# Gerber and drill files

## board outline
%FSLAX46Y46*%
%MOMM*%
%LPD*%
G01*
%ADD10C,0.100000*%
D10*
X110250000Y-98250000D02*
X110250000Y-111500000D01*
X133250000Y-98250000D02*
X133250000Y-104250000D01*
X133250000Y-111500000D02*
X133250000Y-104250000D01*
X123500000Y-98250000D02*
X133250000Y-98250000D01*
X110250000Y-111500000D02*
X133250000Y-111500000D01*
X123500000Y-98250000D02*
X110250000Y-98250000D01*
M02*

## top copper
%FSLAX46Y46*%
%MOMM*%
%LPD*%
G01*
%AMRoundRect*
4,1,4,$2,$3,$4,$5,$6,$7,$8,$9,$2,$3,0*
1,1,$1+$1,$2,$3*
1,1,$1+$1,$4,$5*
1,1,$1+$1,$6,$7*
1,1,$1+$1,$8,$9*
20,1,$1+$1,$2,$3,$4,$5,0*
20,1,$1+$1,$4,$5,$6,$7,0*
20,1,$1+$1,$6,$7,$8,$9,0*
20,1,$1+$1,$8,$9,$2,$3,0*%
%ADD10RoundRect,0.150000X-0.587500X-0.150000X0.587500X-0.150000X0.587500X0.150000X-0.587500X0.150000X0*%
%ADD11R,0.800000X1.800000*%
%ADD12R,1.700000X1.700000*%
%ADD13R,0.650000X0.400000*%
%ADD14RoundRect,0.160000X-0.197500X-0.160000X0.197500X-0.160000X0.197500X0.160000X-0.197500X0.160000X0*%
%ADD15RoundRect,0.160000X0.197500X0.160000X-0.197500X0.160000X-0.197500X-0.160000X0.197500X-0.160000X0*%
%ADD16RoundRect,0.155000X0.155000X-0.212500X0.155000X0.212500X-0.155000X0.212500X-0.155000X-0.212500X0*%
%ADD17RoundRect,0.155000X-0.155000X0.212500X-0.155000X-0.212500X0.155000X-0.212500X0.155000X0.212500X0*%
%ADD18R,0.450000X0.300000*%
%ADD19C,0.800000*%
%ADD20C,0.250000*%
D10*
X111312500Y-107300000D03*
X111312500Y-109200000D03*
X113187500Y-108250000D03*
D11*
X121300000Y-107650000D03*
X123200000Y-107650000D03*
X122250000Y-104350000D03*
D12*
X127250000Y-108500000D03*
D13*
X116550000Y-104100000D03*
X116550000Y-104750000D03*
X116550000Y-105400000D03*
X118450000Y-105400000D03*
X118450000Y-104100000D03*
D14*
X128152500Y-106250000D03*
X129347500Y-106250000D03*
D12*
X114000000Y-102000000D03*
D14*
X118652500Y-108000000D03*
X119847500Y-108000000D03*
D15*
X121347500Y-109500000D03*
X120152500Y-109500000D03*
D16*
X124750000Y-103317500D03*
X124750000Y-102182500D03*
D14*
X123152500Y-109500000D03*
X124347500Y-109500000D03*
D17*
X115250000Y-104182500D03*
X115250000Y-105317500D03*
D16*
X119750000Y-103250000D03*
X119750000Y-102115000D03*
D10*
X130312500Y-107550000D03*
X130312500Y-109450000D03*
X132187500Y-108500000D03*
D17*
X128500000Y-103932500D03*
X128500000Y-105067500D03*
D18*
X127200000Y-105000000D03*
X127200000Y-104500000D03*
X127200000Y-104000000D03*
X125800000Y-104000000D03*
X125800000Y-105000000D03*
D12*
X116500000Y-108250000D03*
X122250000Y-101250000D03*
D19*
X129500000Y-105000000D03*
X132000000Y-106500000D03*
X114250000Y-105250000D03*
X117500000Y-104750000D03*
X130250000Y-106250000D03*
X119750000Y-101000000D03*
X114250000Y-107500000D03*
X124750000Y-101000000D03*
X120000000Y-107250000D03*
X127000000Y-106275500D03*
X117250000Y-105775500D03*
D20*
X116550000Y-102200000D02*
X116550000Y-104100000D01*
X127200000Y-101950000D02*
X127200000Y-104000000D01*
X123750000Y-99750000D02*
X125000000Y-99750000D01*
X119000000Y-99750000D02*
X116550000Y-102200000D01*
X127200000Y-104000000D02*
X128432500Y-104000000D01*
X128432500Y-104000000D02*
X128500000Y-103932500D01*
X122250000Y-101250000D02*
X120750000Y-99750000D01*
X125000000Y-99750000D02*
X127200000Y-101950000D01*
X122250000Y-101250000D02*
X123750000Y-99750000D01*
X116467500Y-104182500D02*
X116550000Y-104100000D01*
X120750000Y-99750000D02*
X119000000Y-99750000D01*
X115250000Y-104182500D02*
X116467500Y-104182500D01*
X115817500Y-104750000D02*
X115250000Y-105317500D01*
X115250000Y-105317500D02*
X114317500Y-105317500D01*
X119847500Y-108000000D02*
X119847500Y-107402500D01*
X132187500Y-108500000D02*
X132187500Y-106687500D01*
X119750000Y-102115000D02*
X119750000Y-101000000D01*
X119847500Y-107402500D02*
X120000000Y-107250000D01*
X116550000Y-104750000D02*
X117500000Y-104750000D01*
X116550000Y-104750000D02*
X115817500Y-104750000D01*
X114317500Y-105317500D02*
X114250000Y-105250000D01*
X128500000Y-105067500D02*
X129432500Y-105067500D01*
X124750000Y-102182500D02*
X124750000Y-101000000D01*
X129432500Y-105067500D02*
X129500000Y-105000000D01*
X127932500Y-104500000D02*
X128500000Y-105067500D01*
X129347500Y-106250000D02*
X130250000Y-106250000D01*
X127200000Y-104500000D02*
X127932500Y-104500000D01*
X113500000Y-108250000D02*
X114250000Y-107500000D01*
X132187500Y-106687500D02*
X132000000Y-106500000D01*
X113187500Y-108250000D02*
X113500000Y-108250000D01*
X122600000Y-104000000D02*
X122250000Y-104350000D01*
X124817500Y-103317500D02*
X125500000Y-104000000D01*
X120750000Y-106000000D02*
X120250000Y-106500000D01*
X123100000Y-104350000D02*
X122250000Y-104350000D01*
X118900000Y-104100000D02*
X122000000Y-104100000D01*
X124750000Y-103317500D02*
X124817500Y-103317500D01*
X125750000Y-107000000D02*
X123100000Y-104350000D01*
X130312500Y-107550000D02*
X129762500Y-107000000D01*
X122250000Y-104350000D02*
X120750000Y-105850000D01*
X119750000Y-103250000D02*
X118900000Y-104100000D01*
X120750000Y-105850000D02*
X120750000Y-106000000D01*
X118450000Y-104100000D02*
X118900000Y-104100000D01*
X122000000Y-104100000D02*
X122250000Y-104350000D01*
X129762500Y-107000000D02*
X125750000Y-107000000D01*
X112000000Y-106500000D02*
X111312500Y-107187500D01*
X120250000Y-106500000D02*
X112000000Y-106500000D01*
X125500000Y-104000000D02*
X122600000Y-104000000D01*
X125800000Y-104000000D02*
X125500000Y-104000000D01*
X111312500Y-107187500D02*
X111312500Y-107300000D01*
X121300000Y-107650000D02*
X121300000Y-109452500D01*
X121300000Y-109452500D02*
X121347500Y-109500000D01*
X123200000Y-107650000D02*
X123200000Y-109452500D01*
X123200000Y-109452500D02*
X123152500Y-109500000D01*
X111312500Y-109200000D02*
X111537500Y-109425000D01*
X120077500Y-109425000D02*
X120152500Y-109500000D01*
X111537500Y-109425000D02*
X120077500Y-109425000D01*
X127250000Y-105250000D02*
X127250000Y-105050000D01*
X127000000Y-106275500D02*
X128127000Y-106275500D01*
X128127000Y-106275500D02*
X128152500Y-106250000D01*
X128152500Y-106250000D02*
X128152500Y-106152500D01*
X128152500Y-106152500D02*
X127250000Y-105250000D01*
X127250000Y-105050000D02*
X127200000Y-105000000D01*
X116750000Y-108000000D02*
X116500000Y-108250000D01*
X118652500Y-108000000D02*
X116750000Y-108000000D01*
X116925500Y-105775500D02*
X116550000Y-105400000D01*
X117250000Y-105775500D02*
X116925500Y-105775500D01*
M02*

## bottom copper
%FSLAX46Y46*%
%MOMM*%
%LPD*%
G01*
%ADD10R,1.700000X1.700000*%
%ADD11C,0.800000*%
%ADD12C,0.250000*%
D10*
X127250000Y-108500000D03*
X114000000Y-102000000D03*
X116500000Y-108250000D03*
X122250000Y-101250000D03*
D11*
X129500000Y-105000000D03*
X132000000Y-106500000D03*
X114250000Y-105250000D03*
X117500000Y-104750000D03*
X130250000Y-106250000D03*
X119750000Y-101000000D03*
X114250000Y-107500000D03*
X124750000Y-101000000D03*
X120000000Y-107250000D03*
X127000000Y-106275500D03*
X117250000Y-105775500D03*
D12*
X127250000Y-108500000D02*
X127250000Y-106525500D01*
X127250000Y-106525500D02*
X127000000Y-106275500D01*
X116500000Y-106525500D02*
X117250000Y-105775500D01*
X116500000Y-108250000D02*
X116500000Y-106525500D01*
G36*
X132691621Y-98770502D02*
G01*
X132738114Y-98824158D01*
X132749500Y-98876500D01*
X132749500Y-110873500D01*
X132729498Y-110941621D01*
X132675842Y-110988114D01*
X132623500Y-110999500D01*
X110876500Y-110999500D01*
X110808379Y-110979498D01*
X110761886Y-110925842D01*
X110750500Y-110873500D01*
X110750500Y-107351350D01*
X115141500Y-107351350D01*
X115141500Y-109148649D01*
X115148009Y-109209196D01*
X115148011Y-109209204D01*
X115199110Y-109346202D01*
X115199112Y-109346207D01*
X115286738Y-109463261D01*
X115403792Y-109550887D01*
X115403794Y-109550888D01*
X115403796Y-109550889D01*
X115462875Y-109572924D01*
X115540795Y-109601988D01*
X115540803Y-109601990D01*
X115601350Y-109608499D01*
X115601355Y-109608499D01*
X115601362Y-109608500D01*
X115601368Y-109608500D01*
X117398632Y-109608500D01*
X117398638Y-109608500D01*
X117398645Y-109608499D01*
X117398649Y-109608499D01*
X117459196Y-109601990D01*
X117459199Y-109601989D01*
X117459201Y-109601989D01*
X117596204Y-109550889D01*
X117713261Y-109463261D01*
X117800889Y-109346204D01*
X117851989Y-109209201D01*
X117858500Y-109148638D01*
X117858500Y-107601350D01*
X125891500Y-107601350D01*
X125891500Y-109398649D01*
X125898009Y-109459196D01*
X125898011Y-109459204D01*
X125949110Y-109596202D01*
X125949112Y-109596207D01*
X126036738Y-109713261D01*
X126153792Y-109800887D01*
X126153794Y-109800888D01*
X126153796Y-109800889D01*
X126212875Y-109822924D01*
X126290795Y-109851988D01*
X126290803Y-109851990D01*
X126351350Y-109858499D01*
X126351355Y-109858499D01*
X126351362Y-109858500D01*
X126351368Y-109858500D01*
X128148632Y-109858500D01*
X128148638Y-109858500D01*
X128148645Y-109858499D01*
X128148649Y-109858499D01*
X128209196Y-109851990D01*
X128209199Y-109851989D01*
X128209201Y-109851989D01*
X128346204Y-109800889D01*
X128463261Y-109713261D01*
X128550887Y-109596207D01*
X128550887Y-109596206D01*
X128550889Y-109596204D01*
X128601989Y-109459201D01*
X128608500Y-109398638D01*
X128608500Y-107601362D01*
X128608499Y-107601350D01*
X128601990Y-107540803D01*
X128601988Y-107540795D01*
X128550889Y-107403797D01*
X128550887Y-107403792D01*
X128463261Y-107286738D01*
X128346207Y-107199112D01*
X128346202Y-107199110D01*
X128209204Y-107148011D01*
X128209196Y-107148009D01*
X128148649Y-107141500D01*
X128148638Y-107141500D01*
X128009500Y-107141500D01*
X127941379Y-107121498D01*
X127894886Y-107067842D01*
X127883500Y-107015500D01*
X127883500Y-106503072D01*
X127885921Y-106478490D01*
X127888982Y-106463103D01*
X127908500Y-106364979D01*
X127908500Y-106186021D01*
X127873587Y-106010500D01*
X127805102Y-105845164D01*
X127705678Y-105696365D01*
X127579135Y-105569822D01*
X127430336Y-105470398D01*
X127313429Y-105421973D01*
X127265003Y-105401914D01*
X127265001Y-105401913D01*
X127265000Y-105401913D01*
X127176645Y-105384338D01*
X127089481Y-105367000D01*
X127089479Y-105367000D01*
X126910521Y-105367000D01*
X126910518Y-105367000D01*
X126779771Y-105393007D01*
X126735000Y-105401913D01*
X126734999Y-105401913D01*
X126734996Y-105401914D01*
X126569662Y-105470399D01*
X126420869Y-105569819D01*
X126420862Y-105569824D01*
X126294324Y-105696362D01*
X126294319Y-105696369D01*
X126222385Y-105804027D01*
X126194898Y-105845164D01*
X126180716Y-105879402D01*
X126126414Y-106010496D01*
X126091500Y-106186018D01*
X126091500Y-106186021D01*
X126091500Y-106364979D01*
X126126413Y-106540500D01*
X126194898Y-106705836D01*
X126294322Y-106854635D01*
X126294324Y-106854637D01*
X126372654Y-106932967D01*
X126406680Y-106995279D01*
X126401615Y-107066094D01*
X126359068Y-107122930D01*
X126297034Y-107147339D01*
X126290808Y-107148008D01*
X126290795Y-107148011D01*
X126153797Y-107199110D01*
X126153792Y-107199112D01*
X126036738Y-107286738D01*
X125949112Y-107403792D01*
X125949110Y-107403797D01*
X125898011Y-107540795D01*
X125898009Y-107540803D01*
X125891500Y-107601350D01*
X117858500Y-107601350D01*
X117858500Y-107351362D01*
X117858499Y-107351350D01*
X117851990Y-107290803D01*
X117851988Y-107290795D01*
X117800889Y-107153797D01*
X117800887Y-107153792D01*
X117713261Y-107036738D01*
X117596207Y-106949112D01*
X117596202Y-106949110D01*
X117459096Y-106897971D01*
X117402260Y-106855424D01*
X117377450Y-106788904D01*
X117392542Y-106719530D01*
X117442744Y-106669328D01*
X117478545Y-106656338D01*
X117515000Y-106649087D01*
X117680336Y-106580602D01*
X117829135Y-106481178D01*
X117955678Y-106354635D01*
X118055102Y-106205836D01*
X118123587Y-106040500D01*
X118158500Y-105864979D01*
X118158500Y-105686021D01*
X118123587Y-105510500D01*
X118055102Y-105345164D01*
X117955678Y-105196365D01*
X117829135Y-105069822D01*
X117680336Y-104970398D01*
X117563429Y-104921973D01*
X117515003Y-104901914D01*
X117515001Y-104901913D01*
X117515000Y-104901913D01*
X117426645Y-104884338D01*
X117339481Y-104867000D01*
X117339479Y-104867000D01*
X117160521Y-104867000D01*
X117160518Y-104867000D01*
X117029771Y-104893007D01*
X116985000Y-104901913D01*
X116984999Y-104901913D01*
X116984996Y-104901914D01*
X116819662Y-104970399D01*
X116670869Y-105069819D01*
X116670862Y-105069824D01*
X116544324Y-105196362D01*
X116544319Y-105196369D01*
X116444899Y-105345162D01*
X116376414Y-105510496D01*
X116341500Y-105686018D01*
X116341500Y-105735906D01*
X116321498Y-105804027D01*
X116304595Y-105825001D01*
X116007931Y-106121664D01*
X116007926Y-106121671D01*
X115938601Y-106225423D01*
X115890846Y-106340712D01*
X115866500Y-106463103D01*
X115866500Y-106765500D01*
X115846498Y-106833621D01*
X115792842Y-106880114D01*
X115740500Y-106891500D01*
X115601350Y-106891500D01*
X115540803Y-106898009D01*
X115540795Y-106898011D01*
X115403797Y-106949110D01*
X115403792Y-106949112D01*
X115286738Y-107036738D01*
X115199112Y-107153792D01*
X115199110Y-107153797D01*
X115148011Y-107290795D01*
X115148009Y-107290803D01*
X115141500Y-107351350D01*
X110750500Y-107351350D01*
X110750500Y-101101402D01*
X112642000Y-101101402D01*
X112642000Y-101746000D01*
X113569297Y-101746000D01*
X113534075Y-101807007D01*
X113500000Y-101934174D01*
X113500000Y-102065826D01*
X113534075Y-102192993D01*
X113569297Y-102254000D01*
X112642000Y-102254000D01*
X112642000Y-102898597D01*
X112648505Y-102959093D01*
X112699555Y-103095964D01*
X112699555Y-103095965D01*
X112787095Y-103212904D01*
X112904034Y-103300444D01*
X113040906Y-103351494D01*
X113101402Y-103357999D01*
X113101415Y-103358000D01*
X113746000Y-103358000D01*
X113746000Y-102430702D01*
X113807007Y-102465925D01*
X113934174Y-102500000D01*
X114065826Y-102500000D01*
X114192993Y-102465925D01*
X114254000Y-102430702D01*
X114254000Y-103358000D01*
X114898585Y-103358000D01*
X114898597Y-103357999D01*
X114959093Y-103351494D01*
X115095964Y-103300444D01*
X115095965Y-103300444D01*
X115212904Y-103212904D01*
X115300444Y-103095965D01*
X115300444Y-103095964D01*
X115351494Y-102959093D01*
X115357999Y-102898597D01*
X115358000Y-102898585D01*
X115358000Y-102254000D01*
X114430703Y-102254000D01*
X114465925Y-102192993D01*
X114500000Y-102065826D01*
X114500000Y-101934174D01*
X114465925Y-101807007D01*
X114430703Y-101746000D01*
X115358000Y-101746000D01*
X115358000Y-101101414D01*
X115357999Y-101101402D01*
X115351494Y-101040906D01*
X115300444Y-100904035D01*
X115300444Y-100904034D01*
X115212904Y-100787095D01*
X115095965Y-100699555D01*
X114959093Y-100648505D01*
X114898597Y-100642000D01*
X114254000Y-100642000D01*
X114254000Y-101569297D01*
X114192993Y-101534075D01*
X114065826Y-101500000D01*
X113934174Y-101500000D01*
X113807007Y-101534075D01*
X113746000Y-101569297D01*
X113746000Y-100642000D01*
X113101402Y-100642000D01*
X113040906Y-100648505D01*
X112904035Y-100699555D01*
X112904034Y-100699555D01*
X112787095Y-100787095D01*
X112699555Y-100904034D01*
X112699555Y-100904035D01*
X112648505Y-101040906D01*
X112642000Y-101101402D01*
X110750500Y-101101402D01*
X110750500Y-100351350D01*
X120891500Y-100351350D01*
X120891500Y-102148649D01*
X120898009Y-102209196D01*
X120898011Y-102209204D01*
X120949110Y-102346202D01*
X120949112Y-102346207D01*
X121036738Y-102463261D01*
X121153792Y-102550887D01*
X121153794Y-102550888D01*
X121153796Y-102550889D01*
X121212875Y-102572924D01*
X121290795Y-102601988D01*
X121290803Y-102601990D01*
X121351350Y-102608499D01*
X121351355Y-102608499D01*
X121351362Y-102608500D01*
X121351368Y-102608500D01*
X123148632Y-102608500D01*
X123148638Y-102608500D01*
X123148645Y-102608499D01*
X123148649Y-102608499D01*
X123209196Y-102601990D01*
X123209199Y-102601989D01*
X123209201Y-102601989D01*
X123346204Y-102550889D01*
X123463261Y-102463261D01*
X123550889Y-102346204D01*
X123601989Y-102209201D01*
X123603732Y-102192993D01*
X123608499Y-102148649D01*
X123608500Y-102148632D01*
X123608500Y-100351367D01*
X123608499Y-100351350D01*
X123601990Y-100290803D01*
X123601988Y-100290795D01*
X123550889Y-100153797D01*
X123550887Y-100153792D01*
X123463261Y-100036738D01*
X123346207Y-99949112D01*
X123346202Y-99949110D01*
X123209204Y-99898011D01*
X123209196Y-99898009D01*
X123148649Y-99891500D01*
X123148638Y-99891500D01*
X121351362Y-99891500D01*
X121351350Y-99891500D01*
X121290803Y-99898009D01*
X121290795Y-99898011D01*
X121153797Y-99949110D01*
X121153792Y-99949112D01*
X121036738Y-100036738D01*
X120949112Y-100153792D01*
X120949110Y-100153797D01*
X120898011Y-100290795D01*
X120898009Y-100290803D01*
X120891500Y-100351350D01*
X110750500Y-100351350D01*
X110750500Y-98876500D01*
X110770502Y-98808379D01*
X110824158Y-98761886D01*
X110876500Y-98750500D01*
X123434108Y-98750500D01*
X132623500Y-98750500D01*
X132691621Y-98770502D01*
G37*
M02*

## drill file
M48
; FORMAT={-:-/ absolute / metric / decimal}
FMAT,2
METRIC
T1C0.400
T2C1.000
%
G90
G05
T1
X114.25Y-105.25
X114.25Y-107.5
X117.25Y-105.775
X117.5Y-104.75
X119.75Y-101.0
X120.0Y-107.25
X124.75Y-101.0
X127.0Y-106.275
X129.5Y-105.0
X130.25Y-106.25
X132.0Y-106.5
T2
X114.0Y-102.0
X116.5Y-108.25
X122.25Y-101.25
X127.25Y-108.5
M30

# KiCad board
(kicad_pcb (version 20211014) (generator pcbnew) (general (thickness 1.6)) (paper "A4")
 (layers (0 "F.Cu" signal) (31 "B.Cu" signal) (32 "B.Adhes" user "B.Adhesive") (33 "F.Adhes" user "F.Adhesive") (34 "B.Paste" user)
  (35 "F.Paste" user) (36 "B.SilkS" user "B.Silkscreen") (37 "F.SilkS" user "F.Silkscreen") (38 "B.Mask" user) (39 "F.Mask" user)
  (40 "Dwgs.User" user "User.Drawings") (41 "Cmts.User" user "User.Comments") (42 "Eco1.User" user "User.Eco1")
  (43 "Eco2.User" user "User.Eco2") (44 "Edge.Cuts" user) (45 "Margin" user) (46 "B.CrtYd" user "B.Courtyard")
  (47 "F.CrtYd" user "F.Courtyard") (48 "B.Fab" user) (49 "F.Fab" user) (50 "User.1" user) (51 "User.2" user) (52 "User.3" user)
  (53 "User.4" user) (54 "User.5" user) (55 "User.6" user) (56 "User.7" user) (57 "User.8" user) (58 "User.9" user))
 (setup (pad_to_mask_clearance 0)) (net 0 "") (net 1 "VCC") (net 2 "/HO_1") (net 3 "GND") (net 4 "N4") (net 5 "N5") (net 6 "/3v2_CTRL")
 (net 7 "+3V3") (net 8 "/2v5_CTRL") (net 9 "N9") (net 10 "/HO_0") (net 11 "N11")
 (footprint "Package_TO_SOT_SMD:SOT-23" (layer "F.Cu") (at 112.25 108.25)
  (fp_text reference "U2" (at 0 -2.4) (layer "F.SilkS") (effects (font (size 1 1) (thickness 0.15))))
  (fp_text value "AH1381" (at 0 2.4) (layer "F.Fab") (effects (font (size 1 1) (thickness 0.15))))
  (pad "1" smd roundrect (at -0.9375 -0.95) (size 1.475 0.6) (layers "F.Cu" "F.Paste" "F.Mask") (roundrect_rratio 0.25) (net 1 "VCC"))
  (pad "2" smd roundrect (at -0.9375 0.95) (size 1.475 0.6) (layers "F.Cu" "F.Paste" "F.Mask") (roundrect_rratio 0.25) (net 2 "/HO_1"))
  (pad "3" smd roundrect (at 0.9375 0) (size 1.475 0.6) (layers "F.Cu" "F.Paste" "F.Mask") (roundrect_rratio 0.25) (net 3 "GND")))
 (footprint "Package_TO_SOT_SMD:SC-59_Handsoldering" (layer "F.Cu") (at 122.25 106 90)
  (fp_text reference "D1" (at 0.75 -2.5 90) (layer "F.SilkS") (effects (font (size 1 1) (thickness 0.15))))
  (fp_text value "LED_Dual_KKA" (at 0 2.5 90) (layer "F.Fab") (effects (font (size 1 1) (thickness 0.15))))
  (pad "1" smd rect (at -1.65 -0.95 90) (size 1.8 0.8) (layers "F.Cu" "F.Paste" "F.Mask") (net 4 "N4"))
  (pad "2" smd rect (at -1.65 0.95 90) (size 1.8 0.8) (layers "F.Cu" "F.Paste" "F.Mask") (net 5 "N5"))
  (pad "3" smd rect (at 1.65 0 90) (size 1.8 0.8) (layers "F.Cu" "F.Paste" "F.Mask") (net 1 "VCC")))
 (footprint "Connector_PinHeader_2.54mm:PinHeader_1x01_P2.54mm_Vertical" (layer "F.Cu") (at 127.25 108.5)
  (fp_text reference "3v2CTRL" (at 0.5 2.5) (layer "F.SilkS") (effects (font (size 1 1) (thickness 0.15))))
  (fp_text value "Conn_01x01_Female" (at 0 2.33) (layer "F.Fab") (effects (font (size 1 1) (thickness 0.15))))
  (pad "1" thru_hole rect (at 0 0) (size 1.7 1.7) (drill 1) (layers *.Cu *.Mask) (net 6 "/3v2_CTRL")))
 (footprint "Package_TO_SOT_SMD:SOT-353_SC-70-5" (layer "F.Cu") (at 117.5 104.75)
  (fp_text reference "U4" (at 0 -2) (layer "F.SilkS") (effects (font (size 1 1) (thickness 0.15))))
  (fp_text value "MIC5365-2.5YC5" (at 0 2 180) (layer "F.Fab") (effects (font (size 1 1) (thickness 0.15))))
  (pad "1" smd rect (at -0.95 -0.65) (size 0.65 0.4) (layers "F.Cu" "F.Paste" "F.Mask") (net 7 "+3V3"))
  (pad "2" smd rect (at -0.95 0) (size 0.65 0.4) (layers "F.Cu" "F.Paste" "F.Mask") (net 3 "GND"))
  (pad "3" smd rect (at -0.95 0.65) (size 0.65 0.4) (layers "F.Cu" "F.Paste" "F.Mask") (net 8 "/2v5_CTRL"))
  (pad "4" smd rect (at 0.95 0.65) (size 0.65 0.4) (layers "F.Cu" "F.Paste" "F.Mask") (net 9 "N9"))
  (pad "5" smd rect (at 0.95 -0.65) (size 0.65 0.4) (layers "F.Cu" "F.Paste" "F.Mask") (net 1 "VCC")))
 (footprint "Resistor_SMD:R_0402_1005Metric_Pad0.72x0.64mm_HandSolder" (layer "F.Cu") (at 128.75 106.25)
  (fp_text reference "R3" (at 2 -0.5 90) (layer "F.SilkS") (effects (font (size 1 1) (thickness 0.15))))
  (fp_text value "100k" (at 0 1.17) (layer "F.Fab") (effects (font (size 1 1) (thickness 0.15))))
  (pad "1" smd roundrect (at -0.5975 0) (size 0.715 0.64) (layers "F.Cu" "F.Paste" "F.Mask") (roundrect_rratio 0.25) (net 6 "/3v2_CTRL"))
  (pad "2" smd roundrect (at 0.5975 0) (size 0.715 0.64) (layers "F.Cu" "F.Paste" "F.Mask") (roundrect_rratio 0.25) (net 3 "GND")))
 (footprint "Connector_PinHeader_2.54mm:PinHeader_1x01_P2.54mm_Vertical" (layer "F.Cu") (at 114 102)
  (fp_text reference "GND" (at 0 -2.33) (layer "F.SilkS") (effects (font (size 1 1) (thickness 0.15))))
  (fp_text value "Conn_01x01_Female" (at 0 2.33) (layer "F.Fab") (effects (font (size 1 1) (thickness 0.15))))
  (pad "1" thru_hole rect (at 0 0) (size 1.7 1.7) (drill 1) (layers *.Cu *.Mask) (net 3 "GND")))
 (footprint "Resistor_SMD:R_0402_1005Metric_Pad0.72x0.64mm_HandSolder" (layer "F.Cu") (at 119.25 108)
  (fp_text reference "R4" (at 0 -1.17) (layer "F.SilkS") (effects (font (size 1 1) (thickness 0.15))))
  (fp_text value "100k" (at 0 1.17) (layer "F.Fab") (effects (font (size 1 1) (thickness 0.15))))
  (pad "1" smd roundrect (at -0.5975 0) (size 0.715 0.64) (layers "F.Cu" "F.Paste" "F.Mask") (roundrect_rratio 0.25) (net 8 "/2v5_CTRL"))
  (pad "2" smd roundrect (at 0.5975 0) (size 0.715 0.64) (layers "F.Cu" "F.Paste" "F.Mask") (roundrect_rratio 0.25) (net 3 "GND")))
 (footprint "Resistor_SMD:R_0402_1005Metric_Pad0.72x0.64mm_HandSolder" (layer "F.Cu") (at 120.75 109.5 180)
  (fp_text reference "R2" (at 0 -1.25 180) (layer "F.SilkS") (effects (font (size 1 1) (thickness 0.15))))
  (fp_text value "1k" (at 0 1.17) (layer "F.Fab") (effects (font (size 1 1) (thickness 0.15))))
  (pad "1" smd roundrect (at -0.5975 0 180) (size 0.715 0.64) (layers "F.Cu" "F.Paste" "F.Mask") (roundrect_rratio 0.25) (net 4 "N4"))
  (pad "2" smd roundrect (at 0.5975 0 180) (size 0.715 0.64) (layers "F.Cu" "F.Paste" "F.Mask") (roundrect_rratio 0.25) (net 2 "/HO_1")))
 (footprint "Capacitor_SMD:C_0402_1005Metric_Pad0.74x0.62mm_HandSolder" (layer "F.Cu") (at 124.75 102.75 90)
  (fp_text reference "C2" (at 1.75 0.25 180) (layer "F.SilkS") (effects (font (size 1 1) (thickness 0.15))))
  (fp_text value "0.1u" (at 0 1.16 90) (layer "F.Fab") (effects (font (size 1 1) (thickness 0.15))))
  (pad "1" smd roundrect (at -0.5675 0 90) (size 0.735 0.62) (layers "F.Cu" "F.Paste" "F.Mask") (roundrect_rratio 0.25) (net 1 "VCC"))
  (pad "2" smd roundrect (at 0.5675 0 90) (size 0.735 0.62) (layers "F.Cu" "F.Paste" "F.Mask") (roundrect_rratio 0.25) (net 3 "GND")))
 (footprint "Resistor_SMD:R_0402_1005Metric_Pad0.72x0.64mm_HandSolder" (layer "F.Cu") (at 123.75 109.5)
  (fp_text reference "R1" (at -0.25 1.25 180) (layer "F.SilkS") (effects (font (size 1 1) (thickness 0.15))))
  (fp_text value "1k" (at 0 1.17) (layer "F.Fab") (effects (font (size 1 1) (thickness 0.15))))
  (pad "1" smd roundrect (at -0.5975 0) (size 0.715 0.64) (layers "F.Cu" "F.Paste" "F.Mask") (roundrect_rratio 0.25) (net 5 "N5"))
  (pad "2" smd roundrect (at 0.5975 0) (size 0.715 0.64) (layers "F.Cu" "F.Paste" "F.Mask") (roundrect_rratio 0.25) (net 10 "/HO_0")))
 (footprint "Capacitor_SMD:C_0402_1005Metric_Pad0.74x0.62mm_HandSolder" (layer "F.Cu") (at 115.25 104.75 -90)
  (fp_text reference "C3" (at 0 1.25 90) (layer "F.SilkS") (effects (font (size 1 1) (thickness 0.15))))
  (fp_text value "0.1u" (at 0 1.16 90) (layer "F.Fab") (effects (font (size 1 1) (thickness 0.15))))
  (pad "1" smd roundrect (at -0.5675 0 270) (size 0.735 0.62) (layers "F.Cu" "F.Paste" "F.Mask") (roundrect_rratio 0.25) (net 7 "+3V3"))
  (pad "2" smd roundrect (at 0.5675 0 270) (size 0.735 0.62) (layers "F.Cu" "F.Paste" "F.Mask") (roundrect_rratio 0.25) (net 3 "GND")))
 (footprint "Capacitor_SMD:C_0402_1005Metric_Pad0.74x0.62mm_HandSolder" (layer "F.Cu") (at 119.75 102.6825 90)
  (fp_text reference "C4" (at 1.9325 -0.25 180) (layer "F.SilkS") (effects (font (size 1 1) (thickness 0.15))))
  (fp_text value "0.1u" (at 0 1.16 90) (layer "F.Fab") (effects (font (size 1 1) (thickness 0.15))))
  (pad "1" smd roundrect (at -0.5675 0 90) (size 0.735 0.62) (layers "F.Cu" "F.Paste" "F.Mask") (roundrect_rratio 0.25) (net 1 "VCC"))
  (pad "2" smd roundrect (at 0.5675 0 90) (size 0.735 0.62) (layers "F.Cu" "F.Paste" "F.Mask") (roundrect_rratio 0.25) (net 3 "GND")))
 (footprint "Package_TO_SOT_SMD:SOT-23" (layer "F.Cu") (at 131.25 108.5)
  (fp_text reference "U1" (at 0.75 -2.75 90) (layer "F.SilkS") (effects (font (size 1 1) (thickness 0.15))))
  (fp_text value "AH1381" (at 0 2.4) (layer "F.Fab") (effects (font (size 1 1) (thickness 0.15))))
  (pad "1" smd roundrect (at -0.9375 -0.95) (size 1.475 0.6) (layers "F.Cu" "F.Paste" "F.Mask") (roundrect_rratio 0.25) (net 1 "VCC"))
  (pad "2" smd roundrect (at -0.9375 0.95) (size 1.475 0.6) (layers "F.Cu" "F.Paste" "F.Mask") (roundrect_rratio 0.25) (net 10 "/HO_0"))
  (pad "3" smd roundrect (at 0.9375 0) (size 1.475 0.6) (layers "F.Cu" "F.Paste" "F.Mask") (roundrect_rratio 0.25) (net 3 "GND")))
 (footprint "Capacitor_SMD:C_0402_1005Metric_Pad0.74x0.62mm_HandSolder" (layer "F.Cu") (at 128.5 104.5 -90)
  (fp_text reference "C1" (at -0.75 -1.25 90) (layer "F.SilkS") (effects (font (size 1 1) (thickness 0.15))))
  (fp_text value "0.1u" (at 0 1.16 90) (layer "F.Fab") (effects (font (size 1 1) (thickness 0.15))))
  (pad "1" smd roundrect (at -0.5675 0 270) (size 0.735 0.62) (layers "F.Cu" "F.Paste" "F.Mask") (roundrect_rratio 0.25) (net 7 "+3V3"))
  (pad "2" smd roundrect (at 0.5675 0 270) (size 0.735 0.62) (layers "F.Cu" "F.Paste" "F.Mask") (roundrect_rratio 0.25) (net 3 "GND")))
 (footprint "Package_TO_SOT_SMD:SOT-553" (layer "F.Cu") (at 126.5 104.5 180)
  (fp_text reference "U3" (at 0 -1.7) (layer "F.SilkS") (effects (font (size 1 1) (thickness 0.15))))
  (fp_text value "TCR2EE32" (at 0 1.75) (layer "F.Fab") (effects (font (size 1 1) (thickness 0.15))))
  (pad "1" smd rect (at -0.7 -0.5 180) (size 0.45 0.3) (layers "F.Cu" "F.Paste" "F.Mask") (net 6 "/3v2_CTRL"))
  (pad "2" smd rect (at -0.7 0 180) (size 0.45 0.3) (layers "F.Cu" "F.Paste" "F.Mask") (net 3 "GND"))
  (pad "3" smd rect (at -0.7 0.5 180) (size 0.45 0.3) (layers "F.Cu" "F.Paste" "F.Mask") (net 7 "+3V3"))
  (pad "4" smd rect (at 0.7 0.5 180) (size 0.45 0.3) (layers "F.Cu" "F.Paste" "F.Mask") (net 1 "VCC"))
  (pad "5" smd rect (at 0.7 -0.5 180) (size 0.45 0.3) (layers "F.Cu" "F.Paste" "F.Mask") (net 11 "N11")))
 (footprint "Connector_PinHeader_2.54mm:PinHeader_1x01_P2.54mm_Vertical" (layer "F.Cu") (at 116.5 108.25)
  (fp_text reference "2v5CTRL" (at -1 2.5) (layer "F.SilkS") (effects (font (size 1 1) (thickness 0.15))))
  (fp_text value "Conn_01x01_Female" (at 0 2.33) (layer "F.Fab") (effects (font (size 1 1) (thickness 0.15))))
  (pad "1" thru_hole rect (at 0 0) (size 1.7 1.7) (drill 1) (layers *.Cu *.Mask) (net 8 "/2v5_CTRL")))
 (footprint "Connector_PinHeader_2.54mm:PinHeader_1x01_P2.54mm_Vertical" (layer "F.Cu") (at 122.25 101.25)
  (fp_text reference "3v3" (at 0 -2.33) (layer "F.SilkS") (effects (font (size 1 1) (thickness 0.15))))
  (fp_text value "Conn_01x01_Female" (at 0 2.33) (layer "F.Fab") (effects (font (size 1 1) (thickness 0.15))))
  (pad "1" thru_hole rect (at 0 0) (size 1.7 1.7) (drill 1) (layers *.Cu *.Mask) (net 7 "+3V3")))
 (gr_line (start 110.25 98.25) (end 110.25 111.5) (layer "Edge.Cuts") (width 0.1))
 (gr_line (start 133.25 98.25) (end 133.25 104.25) (layer "Edge.Cuts") (width 0.1))
 (gr_line (start 133.25 111.5) (end 133.25 104.25) (layer "Edge.Cuts") (width 0.1))
 (gr_line (start 123.5 98.25) (end 133.25 98.25) (layer "Edge.Cuts") (width 0.1))
 (gr_line (start 110.25 111.5) (end 133.25 111.5) (layer "Edge.Cuts") (width 0.1))
 (gr_line (start 123.5 98.25) (end 110.25 98.25) (layer "Edge.Cuts") (width 0.1))
 (segment (start 116.55 102.2) (end 116.55 104.1) (width 0.25) (layer "F.Cu") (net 7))
 (segment (start 127.2 101.95) (end 127.2 104) (width 0.25) (layer "F.Cu") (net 7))
 (segment (start 123.75 99.75) (end 125 99.75) (width 0.25) (layer "F.Cu") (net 7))
 (segment (start 119 99.75) (end 116.55 102.2) (width 0.25) (layer "F.Cu") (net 7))
 (segment (start 127.2 104) (end 128.4325 104) (width 0.25) (layer "F.Cu") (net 7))
 (segment (start 128.4325 104) (end 128.5 103.9325) (width 0.25) (layer "F.Cu") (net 7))
 (segment (start 122.25 101.25) (end 120.75 99.75) (width 0.25) (layer "F.Cu") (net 7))
 (segment (start 125 99.75) (end 127.2 101.95) (width 0.25) (layer "F.Cu") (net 7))
 (segment (start 122.25 101.25) (end 123.75 99.75) (width 0.25) (layer "F.Cu") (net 7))
 (segment (start 116.4675 104.1825) (end 116.55 104.1) (width 0.25) (layer "F.Cu") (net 7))
 (segment (start 120.75 99.75) (end 119 99.75) (width 0.25) (layer "F.Cu") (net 7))
 (segment (start 115.25 104.1825) (end 116.4675 104.1825) (width 0.25) (layer "F.Cu") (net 7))
 (segment (start 115.8175 104.75) (end 115.25 105.3175) (width 0.25) (layer "F.Cu") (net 3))
 (segment (start 115.25 105.3175) (end 114.3175 105.3175) (width 0.25) (layer "F.Cu") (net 3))
 (segment (start 119.8475 108) (end 119.8475 107.4025) (width 0.25) (layer "F.Cu") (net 3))
 (segment (start 132.1875 108.5) (end 132.1875 106.6875) (width 0.25) (layer "F.Cu") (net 3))
 (segment (start 119.75 102.115) (end 119.75 101) (width 0.25) (layer "F.Cu") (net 3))
 (segment (start 119.8475 107.4025) (end 120 107.25) (width 0.25) (layer "F.Cu") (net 3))
 (segment (start 116.55 104.75) (end 117.5 104.75) (width 0.25) (layer "F.Cu") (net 3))
 (segment (start 116.55 104.75) (end 115.8175 104.75) (width 0.25) (layer "F.Cu") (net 3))
 (segment (start 114.3175 105.3175) (end 114.25 105.25) (width 0.25) (layer "F.Cu") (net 3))
 (segment (start 128.5 105.0675) (end 129.4325 105.0675) (width 0.25) (layer "F.Cu") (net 3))
 (segment (start 124.75 102.1825) (end 124.75 101) (width 0.25) (layer "F.Cu") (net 3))
 (segment (start 129.4325 105.0675) (end 129.5 105) (width 0.25) (layer "F.Cu") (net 3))
 (segment (start 127.9325 104.5) (end 128.5 105.0675) (width 0.25) (layer "F.Cu") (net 3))
 (segment (start 129.3475 106.25) (end 130.25 106.25) (width 0.25) (layer "F.Cu") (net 3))
 (segment (start 127.2 104.5) (end 127.9325 104.5) (width 0.25) (layer "F.Cu") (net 3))
 (segment (start 113.5 108.25) (end 114.25 107.5) (width 0.25) (layer "F.Cu") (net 3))
 (segment (start 132.1875 106.6875) (end 132 106.5) (width 0.25) (layer "F.Cu") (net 3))
 (segment (start 113.1875 108.25) (end 113.5 108.25) (width 0.25) (layer "F.Cu") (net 3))
 (via (at 129.5 105) (size 0.8) (drill 0.4) (layers "F.Cu" "B.Cu") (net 3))
 (via (at 132 106.5) (size 0.8) (drill 0.4) (layers "F.Cu" "B.Cu") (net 3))
 (via (at 114.25 105.25) (size 0.8) (drill 0.4) (layers "F.Cu" "B.Cu") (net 3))
 (via (at 117.5 104.75) (size 0.8) (drill 0.4) (layers "F.Cu" "B.Cu") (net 3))
 (via (at 130.25 106.25) (size 0.8) (drill 0.4) (layers "F.Cu" "B.Cu") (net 3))
 (via (at 119.75 101) (size 0.8) (drill 0.4) (layers "F.Cu" "B.Cu") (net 3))
 (via (at 114.25 107.5) (size 0.8) (drill 0.4) (layers "F.Cu" "B.Cu") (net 3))
 (via (at 124.75 101) (size 0.8) (drill 0.4) (layers "F.Cu" "B.Cu") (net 3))
 (via (at 120 107.25) (size 0.8) (drill 0.4) (layers "F.Cu" "B.Cu") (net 3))
 (segment (start 122.6 104) (end 122.25 104.35) (width 0.25) (layer "F.Cu") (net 1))
 (segment (start 124.8175 103.3175) (end 125.5 104) (width 0.25) (layer "F.Cu") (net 1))
 (segment (start 120.75 106) (end 120.25 106.5) (width 0.25) (layer "F.Cu") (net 1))
 (segment (start 123.1 104.35) (end 122.25 104.35) (width 0.25) (layer "F.Cu") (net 1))
 (segment (start 118.9 104.1) (end 122 104.1) (width 0.25) (layer "F.Cu") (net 1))
 (segment (start 124.75 103.3175) (end 124.8175 103.3175) (width 0.25) (layer "F.Cu") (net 1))
 (segment (start 125.75 107) (end 123.1 104.35) (width 0.25) (layer "F.Cu") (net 1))
 (segment (start 130.3125 107.55) (end 129.7625 107) (width 0.25) (layer "F.Cu") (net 1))
 (segment (start 122.25 104.35) (end 120.75 105.85) (width 0.25) (layer "F.Cu") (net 1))
 (segment (start 119.75 103.25) (end 118.9 104.1) (width 0.25) (layer "F.Cu") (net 1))
 (segment (start 120.75 105.85) (end 120.75 106) (width 0.25) (layer "F.Cu") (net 1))
 (segment (start 118.45 104.1) (end 118.9 104.1) (width 0.25) (layer "F.Cu") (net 1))
 (segment (start 122 104.1) (end 122.25 104.35) (width 0.25) (layer "F.Cu") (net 1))
 (segment (start 129.7625 107) (end 125.75 107) (width 0.25) (layer "F.Cu") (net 1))
 (segment (start 112 106.5) (end 111.3125 107.1875) (width 0.25) (layer "F.Cu") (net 1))
 (segment (start 120.25 106.5) (end 112 106.5) (width 0.25) (layer "F.Cu") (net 1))
 (segment (start 125.5 104) (end 122.6 104) (width 0.25) (layer "F.Cu") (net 1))
 (segment (start 125.8 104) (end 125.5 104) (width 0.25) (layer "F.Cu") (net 1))
 (segment (start 111.3125 107.1875) (end 111.3125 107.3) (width 0.25) (layer "F.Cu") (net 1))
 (segment (start 121.3 107.65) (end 121.3 109.4525) (width 0.25) (layer "F.Cu") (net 4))
 (segment (start 121.3 109.4525) (end 121.3475 109.5) (width 0.25) (layer "F.Cu") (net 4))
 (segment (start 123.2 107.65) (end 123.2 109.4525) (width 0.25) (layer "F.Cu") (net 5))
 (segment (start 123.2 109.4525) (end 123.1525 109.5) (width 0.25) (layer "F.Cu") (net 5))
 (segment (start 111.3125 109.2) (end 111.5375 109.425) (width 0.25) (layer "F.Cu") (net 2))
 (segment (start 120.0775 109.425) (end 120.1525 109.5) (width 0.25) (layer "F.Cu") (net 2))
 (segment (start 111.5375 109.425) (end 120.0775 109.425) (width 0.25) (layer "F.Cu") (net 2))
 (segment (start 127.25 105.25) (end 127.25 105.05) (width 0.25) (layer "F.Cu") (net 6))
 (segment (start 127 106.2755) (end 128.127 106.2755) (width 0.25) (layer "F.Cu") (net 6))
 (segment (start 128.127 106.2755) (end 128.1525 106.25) (width 0.25) (layer "F.Cu") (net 6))
 (segment (start 128.1525 106.25) (end 128.1525 106.1525) (width 0.25) (layer "F.Cu") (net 6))
 (segment (start 128.1525 106.1525) (end 127.25 105.25) (width 0.25) (layer "F.Cu") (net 6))
 (segment (start 127.25 105.05) (end 127.2 105) (width 0.25) (layer "F.Cu") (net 6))
 (via (at 127 106.2755) (size 0.8) (drill 0.4) (layers "F.Cu" "B.Cu") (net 6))
 (segment (start 127.25 108.5) (end 127.25 106.5255) (width 0.25) (layer "B.Cu") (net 6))
 (segment (start 127.25 106.5255) (end 127 106.2755) (width 0.25) (layer "B.Cu") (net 6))
 (segment (start 116.75 108) (end 116.5 108.25) (width 0.25) (layer "F.Cu") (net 8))
 (segment (start 118.6525 108) (end 116.75 108) (width 0.25) (layer "F.Cu") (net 8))
 (segment (start 116.9255 105.7755) (end 116.55 105.4) (width 0.25) (layer "F.Cu") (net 8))
 (segment (start 117.25 105.7755) (end 116.9255 105.7755) (width 0.25) (layer "F.Cu") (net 8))
 (via (at 117.25 105.7755) (size 0.8) (drill 0.4) (layers "F.Cu" "B.Cu") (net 8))
 (segment (start 116.5 106.5255) (end 117.25 105.7755) (width 0.25) (layer "B.Cu") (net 8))
 (segment (start 116.5 108.25) (end 116.5 106.5255) (width 0.25) (layer "B.Cu") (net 8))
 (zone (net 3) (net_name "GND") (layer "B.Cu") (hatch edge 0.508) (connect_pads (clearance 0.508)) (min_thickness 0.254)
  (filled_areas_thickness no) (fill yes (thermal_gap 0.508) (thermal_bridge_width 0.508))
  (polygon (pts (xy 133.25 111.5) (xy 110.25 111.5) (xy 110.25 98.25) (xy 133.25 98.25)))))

